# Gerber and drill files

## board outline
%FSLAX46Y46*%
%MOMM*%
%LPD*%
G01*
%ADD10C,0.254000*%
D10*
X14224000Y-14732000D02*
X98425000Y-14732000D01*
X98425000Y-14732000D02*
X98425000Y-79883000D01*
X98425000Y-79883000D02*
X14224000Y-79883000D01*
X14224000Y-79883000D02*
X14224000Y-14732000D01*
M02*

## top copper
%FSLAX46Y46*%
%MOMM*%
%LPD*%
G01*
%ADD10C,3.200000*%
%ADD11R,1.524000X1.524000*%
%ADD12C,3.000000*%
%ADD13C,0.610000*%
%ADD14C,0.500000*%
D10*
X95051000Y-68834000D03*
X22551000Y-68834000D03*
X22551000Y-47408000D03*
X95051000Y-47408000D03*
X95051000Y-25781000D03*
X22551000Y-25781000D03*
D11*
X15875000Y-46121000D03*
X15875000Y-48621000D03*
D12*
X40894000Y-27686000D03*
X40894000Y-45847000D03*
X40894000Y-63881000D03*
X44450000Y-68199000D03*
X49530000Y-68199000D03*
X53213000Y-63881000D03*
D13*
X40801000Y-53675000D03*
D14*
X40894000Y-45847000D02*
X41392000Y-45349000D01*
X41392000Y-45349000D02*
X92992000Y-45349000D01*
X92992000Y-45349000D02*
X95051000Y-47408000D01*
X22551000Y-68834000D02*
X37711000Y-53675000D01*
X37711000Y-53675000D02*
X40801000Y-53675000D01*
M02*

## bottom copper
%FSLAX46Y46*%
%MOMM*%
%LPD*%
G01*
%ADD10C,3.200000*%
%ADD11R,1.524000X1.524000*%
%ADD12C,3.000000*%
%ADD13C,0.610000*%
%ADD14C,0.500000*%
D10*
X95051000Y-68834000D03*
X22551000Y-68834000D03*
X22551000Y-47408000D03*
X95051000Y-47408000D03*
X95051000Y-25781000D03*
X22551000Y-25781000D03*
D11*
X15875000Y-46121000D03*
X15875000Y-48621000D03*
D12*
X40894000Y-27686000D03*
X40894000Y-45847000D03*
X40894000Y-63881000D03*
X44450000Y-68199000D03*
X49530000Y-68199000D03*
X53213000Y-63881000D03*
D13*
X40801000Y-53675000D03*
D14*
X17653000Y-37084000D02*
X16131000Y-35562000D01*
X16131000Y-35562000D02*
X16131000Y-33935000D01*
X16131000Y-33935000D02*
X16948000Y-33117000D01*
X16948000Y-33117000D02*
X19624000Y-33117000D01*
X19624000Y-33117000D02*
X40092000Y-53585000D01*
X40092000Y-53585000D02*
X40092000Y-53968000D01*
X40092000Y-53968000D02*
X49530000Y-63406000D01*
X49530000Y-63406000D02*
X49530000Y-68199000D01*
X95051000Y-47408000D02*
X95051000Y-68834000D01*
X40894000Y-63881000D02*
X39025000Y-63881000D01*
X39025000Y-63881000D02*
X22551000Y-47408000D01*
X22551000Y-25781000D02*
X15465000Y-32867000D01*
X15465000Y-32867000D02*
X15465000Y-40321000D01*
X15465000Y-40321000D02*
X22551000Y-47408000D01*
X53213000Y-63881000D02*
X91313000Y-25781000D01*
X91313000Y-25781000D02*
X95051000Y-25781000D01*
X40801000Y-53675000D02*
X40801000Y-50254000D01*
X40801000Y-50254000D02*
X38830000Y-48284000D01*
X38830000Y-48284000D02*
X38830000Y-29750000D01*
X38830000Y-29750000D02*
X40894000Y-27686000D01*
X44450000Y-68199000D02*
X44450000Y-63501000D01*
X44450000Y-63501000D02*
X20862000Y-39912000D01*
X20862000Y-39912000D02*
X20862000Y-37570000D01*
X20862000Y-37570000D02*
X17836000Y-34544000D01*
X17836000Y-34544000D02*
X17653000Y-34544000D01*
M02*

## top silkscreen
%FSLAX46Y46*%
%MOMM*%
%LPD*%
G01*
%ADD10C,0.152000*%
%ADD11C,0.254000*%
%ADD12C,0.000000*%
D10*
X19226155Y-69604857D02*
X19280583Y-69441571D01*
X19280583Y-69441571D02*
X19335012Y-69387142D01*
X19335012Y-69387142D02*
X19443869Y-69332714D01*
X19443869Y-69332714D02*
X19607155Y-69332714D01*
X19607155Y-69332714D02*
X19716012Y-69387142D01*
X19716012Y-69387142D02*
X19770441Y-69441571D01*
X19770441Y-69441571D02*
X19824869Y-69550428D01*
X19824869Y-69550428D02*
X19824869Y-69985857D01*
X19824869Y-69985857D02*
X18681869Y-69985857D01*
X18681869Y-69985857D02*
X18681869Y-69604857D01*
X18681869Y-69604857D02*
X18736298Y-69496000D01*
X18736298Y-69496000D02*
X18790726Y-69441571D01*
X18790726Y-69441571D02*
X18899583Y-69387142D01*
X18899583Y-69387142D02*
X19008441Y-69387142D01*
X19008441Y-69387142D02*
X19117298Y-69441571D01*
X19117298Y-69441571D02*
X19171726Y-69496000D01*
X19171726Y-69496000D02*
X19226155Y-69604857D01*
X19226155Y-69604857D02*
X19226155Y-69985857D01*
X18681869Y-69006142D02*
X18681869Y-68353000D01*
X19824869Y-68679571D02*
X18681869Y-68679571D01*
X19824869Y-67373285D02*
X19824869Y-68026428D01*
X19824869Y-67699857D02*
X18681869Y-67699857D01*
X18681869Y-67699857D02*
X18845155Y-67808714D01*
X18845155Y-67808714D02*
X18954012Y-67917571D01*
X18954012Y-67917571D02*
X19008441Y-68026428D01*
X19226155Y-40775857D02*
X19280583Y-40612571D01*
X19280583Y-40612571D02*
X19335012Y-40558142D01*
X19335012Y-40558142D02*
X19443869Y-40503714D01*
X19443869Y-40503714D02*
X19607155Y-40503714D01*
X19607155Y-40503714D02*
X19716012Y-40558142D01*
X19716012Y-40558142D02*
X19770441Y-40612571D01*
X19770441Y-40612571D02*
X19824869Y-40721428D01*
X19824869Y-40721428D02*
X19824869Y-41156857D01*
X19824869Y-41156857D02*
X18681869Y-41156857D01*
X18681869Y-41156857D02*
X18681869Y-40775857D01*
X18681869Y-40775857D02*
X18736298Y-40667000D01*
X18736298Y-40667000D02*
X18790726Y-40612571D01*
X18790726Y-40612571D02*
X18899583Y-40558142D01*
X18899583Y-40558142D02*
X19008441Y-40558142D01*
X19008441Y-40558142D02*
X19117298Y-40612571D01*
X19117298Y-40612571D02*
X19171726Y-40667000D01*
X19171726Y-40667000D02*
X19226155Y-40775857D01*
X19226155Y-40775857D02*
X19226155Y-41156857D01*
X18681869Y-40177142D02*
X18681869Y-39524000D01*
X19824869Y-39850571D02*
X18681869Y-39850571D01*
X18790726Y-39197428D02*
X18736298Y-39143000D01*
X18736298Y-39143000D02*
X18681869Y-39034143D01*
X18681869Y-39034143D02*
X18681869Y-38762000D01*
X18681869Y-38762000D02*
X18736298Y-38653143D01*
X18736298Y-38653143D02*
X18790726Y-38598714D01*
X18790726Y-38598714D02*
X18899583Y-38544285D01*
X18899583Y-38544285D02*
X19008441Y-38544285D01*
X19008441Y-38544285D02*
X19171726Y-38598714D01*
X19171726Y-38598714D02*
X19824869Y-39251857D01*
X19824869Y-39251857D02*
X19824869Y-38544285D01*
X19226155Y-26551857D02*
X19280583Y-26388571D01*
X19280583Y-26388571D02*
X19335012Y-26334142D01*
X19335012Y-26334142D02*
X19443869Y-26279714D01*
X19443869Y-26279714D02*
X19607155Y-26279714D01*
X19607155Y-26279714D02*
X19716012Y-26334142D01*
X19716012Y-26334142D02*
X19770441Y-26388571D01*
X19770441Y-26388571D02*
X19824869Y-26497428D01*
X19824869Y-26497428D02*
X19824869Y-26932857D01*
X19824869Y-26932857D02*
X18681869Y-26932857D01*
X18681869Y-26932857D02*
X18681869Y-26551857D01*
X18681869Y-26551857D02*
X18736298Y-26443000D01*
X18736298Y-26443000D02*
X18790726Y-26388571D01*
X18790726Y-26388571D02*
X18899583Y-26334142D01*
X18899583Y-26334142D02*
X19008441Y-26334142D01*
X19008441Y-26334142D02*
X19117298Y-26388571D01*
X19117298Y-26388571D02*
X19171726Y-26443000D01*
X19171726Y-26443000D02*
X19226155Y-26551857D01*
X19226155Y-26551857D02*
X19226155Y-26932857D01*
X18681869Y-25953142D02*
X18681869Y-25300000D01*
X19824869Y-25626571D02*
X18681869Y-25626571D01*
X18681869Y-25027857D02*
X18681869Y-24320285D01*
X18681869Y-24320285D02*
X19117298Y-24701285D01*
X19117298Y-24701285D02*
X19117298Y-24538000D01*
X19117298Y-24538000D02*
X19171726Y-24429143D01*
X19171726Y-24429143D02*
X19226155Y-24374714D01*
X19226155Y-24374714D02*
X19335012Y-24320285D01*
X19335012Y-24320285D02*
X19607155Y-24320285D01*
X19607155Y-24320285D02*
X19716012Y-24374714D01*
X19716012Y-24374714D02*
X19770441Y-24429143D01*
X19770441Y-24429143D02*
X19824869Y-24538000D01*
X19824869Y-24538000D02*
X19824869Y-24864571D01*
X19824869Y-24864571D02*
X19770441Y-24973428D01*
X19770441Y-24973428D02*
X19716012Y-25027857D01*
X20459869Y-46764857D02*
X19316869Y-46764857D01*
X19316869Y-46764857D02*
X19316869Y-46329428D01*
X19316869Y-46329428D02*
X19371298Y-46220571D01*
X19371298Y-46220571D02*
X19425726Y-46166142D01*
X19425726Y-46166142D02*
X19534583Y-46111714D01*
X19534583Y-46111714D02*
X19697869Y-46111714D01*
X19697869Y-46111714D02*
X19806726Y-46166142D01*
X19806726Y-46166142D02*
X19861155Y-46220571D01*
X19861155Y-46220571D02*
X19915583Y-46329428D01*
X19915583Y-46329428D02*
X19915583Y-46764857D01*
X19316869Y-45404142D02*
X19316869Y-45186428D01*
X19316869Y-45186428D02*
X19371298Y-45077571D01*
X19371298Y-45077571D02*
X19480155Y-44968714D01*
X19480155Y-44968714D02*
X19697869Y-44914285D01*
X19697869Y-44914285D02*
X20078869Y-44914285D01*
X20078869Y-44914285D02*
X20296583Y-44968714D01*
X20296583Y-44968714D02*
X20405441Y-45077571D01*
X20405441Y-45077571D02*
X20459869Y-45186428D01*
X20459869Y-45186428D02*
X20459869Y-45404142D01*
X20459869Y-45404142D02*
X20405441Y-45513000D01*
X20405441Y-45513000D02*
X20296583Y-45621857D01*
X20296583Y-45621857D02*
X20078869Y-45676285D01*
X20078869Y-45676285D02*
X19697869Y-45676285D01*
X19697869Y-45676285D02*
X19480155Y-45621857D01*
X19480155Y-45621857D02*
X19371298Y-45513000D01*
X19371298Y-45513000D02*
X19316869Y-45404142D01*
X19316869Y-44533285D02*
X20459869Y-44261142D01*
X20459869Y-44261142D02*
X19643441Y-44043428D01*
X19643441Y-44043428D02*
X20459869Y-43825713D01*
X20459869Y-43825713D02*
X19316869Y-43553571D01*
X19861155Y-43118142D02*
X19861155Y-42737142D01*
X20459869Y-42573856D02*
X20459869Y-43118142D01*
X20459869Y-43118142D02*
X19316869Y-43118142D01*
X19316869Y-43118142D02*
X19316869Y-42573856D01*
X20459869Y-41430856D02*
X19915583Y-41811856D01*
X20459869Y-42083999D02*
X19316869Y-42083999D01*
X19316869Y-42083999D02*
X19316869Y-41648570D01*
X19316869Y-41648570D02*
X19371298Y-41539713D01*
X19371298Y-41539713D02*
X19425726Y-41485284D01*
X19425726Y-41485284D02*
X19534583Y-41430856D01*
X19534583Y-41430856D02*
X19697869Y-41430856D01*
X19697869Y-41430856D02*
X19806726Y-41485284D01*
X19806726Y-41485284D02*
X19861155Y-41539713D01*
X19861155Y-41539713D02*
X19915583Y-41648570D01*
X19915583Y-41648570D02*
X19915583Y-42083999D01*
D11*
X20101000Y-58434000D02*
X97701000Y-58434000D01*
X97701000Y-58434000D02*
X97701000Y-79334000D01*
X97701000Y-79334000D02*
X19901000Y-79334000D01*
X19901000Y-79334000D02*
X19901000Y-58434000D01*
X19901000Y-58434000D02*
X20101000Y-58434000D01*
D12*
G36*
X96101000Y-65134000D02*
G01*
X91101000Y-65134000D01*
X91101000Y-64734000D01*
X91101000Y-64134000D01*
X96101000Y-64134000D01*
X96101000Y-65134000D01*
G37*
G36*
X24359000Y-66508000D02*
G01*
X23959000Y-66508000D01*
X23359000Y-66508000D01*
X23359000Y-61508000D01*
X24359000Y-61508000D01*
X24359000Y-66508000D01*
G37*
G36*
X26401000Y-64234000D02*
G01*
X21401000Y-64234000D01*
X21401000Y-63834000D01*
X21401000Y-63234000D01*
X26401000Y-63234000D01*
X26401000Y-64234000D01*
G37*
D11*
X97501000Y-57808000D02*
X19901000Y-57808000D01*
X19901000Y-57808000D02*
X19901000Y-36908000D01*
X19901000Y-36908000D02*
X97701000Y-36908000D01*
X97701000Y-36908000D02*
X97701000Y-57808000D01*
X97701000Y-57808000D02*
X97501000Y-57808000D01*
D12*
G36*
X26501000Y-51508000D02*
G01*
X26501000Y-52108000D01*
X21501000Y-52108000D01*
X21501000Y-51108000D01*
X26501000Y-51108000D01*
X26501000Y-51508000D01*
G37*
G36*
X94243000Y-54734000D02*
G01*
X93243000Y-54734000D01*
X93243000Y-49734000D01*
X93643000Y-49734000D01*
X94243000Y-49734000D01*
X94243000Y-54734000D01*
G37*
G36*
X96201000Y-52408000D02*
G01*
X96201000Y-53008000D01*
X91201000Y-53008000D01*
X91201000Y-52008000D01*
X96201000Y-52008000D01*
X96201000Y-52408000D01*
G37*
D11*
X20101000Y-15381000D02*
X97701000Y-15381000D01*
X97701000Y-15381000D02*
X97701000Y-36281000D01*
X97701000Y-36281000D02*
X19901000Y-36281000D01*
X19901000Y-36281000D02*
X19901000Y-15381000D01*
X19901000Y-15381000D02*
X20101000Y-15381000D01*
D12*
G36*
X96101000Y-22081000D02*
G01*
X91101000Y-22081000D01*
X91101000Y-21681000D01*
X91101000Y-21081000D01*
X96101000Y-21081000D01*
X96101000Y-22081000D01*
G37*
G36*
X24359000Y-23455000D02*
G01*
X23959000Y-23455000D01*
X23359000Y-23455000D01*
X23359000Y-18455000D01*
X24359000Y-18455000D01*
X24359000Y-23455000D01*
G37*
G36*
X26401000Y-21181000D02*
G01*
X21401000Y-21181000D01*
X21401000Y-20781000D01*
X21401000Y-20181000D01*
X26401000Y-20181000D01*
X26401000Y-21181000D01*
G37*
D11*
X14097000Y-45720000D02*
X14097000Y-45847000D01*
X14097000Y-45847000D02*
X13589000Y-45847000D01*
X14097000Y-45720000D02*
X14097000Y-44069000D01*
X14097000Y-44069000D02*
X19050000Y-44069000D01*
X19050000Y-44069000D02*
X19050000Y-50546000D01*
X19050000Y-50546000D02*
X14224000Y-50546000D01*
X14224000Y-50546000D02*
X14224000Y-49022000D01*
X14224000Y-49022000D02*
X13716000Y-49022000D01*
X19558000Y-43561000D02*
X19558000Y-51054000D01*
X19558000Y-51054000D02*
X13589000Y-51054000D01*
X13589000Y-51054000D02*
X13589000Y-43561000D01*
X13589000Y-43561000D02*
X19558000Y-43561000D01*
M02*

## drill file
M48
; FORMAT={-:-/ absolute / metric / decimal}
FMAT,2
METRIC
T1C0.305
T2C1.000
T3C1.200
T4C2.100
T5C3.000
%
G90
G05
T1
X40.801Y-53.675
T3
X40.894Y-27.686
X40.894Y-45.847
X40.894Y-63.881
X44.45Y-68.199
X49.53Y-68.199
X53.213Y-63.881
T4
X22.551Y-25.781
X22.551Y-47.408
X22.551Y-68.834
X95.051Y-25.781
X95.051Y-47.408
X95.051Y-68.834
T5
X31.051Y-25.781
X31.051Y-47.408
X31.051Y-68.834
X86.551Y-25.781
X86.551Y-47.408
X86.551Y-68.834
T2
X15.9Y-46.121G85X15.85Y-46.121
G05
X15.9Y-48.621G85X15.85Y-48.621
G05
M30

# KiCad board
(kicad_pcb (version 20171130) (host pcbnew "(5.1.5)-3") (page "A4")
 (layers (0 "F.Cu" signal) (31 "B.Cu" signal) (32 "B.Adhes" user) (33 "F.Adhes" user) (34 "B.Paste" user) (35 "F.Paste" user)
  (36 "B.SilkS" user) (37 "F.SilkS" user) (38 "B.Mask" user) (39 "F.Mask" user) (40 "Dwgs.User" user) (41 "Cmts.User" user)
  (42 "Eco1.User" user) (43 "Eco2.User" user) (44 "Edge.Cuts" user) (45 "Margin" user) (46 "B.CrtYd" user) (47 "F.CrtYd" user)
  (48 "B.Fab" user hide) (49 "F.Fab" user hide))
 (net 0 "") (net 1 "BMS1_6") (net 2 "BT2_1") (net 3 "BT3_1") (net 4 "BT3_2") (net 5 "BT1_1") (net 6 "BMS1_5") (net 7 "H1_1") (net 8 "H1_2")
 (segment (start 17.653 37.084) (end 16.131 35.562) (width 0.5) (layer "B.Cu") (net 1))
 (segment (start 16.131 35.562) (end 16.131 33.935) (width 0.5) (layer "B.Cu") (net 1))
 (segment (start 16.131 33.935) (end 16.948 33.117) (width 0.5) (layer "B.Cu") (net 1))
 (segment (start 16.948 33.117) (end 19.624 33.117) (width 0.5) (layer "B.Cu") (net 1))
 (segment (start 19.624 33.117) (end 40.092 53.585) (width 0.5) (layer "B.Cu") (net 1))
 (segment (start 40.092 53.585) (end 40.092 53.968) (width 0.5) (layer "B.Cu") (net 1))
 (segment (start 40.092 53.968) (end 49.53 63.406) (width 0.5) (layer "B.Cu") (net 1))
 (segment (start 49.53 63.406) (end 49.53 68.199) (width 0.5) (layer "B.Cu") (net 1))
 (segment (start 95.051 47.408) (end 95.051 68.834) (width 0.5) (layer "B.Cu") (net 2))
 (segment (start 40.894 63.881) (end 39.025 63.881) (width 0.5) (layer "B.Cu") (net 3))
 (segment (start 39.025 63.881) (end 22.551 47.408) (width 0.5) (layer "B.Cu") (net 3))
 (segment (start 22.551 25.781) (end 15.465 32.867) (width 0.5) (layer "B.Cu") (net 3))
 (segment (start 15.465 32.867) (end 15.465 40.321) (width 0.5) (layer "B.Cu") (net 3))
 (segment (start 15.465 40.321) (end 22.551 47.408) (width 0.5) (layer "B.Cu") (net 3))
 (segment (start 53.213 63.881) (end 91.313 25.781) (width 0.5) (layer "B.Cu") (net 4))
 (segment (start 91.313 25.781) (end 95.051 25.781) (width 0.5) (layer "B.Cu") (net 4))
 (segment (start 40.801 53.675) (end 40.801 50.254) (width 0.5) (layer "B.Cu") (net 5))
 (segment (start 40.801 50.254) (end 38.83 48.284) (width 0.5) (layer "B.Cu") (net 5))
 (segment (start 38.83 48.284) (end 38.83 29.75) (width 0.5) (layer "B.Cu") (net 5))
 (segment (start 38.83 29.75) (end 40.894 27.686) (width 0.5) (layer "B.Cu") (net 5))
 (segment (start 44.45 68.199) (end 44.45 63.501) (width 0.5) (layer "B.Cu") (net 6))
 (segment (start 44.45 63.501) (end 20.862 39.912) (width 0.5) (layer "B.Cu") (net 6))
 (segment (start 20.862 39.912) (end 20.862 37.57) (width 0.5) (layer "B.Cu") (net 6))
 (segment (start 20.862 37.57) (end 17.836 34.544) (width 0.5) (layer "B.Cu") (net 6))
 (segment (start 17.836 34.544) (end 17.653 34.544) (width 0.5) (layer "B.Cu") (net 6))
 (gr_line (start 14.224 14.732) (end 98.425 14.732) (width 0.254) (layer "Edge.Cuts"))
 (gr_line (start 98.425 14.732) (end 98.425 79.883) (width 0.254) (layer "Edge.Cuts"))
 (gr_line (start 98.425 79.883) (end 14.224 79.883) (width 0.254) (layer "Edge.Cuts"))
 (gr_line (start 14.224 79.883) (end 14.224 14.732) (width 0.254) (layer "Edge.Cuts"))
 (segment (start 40.894 45.847) (end 41.392 45.349) (width 0.5) (layer "F.Cu") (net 2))
 (segment (start 41.392 45.349) (end 92.992 45.349) (width 0.5) (layer "F.Cu") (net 2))
 (segment (start 92.992 45.349) (end 95.051 47.408) (width 0.5) (layer "F.Cu") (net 2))
 (segment (start 22.551 68.834) (end 37.711 53.675) (width 0.5) (layer "F.Cu") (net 5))
 (segment (start 37.711 53.675) (end 40.801 53.675) (width 0.5) (layer "F.Cu") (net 5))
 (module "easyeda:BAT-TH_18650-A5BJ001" (layer "F.Cu") (at 58.801 68.834)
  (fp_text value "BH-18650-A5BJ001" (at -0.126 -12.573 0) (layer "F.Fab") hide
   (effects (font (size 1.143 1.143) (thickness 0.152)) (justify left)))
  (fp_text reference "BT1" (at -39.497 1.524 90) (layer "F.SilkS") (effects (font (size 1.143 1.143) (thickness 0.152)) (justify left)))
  (fp_line (start -38.7 -10.4) (end 38.9 -10.4) (width 0.254) (layer "F.SilkS"))
  (fp_line (start 38.9 -10.4) (end 38.9 10.5) (width 0.254) (layer "F.SilkS"))
  (fp_line (start 38.9 10.5) (end -38.9 10.5) (width 0.254) (layer "F.SilkS"))
  (fp_line (start -38.9 10.5) (end -38.9 -10.4) (width 0.254) (layer "F.SilkS"))
  (fp_line (start -38.9 -10.4) (end -38.7 -10.4) (width 0.254) (layer "F.SilkS"))
  (fp_poly (pts (xy 32.3 -4.7) (xy 37.3 -4.7) (xy 37.3 -3.7) (xy 32.3 -3.7) (xy 32.3 -4.1)) (layer "F.SilkS") (width 0))
  (fp_poly
   (pts (xy -35.442 -2.326) (xy -35.442 -7.326) (xy -34.442 -7.326) (xy -34.442 -2.326) (xy -34.842 -2.326)) (layer "F.SilkS") (width 0))
  (fp_poly (pts (xy -37.4 -5.6) (xy -32.4 -5.6) (xy -32.4 -4.6) (xy -37.4 -4.6) (xy -37.4 -5)) (layer "F.SilkS") (width 0))
  (pad "" np_thru_hole circle (at 27.75 0) (size 3 3) (drill 3) (layers "*.Cu" "*.Mask"))
  (pad "" np_thru_hole circle (at -27.75 0) (size 3 3) (drill 3) (layers "*.Cu" "*.Mask"))
  (pad 2 thru_hole circle (at 36.25 0 0) (size 3.2 3.2) (layers "*.Cu" "*.Paste" "*.Mask") (drill 2.1) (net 2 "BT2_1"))
  (pad 1 thru_hole circle (at -36.25 0 0) (size 3.2 3.2) (layers "*.Cu" "*.Paste" "*.Mask") (drill 2.1) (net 5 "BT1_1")))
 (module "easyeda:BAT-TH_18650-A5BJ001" (layer "F.Cu") (at 58.801 47.408 180)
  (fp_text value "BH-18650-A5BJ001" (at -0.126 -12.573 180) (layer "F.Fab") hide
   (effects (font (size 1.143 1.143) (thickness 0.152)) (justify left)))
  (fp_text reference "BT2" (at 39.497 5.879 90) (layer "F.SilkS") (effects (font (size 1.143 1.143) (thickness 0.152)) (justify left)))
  (fp_line (start -38.7 -10.4) (end 38.9 -10.4) (width 0.254) (layer "F.SilkS"))
  (fp_line (start 38.9 -10.4) (end 38.9 10.5) (width 0.254) (layer "F.SilkS"))
  (fp_line (start 38.9 10.5) (end -38.9 10.5) (width 0.254) (layer "F.SilkS"))
  (fp_line (start -38.9 10.5) (end -38.9 -10.4) (width 0.254) (layer "F.SilkS"))
  (fp_line (start -38.9 -10.4) (end -38.7 -10.4) (width 0.254) (layer "F.SilkS"))
  (fp_poly (pts (xy 32.3 -4.7) (xy 37.3 -4.7) (xy 37.3 -3.7) (xy 32.3 -3.7) (xy 32.3 -4.1)) (layer "F.SilkS") (width 0))
  (fp_poly
   (pts (xy -35.442 -2.326) (xy -35.442 -7.326) (xy -34.442 -7.326) (xy -34.442 -2.326) (xy -34.842 -2.326)) (layer "F.SilkS") (width 0))
  (fp_poly (pts (xy -37.4 -5.6) (xy -32.4 -5.6) (xy -32.4 -4.6) (xy -37.4 -4.6) (xy -37.4 -5)) (layer "F.SilkS") (width 0))
  (pad "" np_thru_hole circle (at 27.75 0) (size 3 3) (drill 3) (layers "*.Cu" "*.Mask"))
  (pad "" np_thru_hole circle (at -27.75 0) (size 3 3) (drill 3) (layers "*.Cu" "*.Mask"))
  (pad 2 thru_hole circle (at 36.25 0 180) (size 3.2 3.2) (layers "*.Cu" "*.Paste" "*.Mask") (drill 2.1) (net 3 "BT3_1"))
  (pad 1 thru_hole circle (at -36.25 0 180) (size 3.2 3.2) (layers "*.Cu" "*.Paste" "*.Mask") (drill 2.1) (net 2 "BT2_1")))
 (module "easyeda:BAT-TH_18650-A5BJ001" (layer "F.Cu") (at 58.801 25.781)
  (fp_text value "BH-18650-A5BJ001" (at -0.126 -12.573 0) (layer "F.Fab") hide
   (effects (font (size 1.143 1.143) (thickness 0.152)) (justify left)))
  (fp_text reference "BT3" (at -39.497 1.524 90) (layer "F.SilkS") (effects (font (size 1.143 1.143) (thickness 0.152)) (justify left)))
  (fp_line (start -38.7 -10.4) (end 38.9 -10.4) (width 0.254) (layer "F.SilkS"))
  (fp_line (start 38.9 -10.4) (end 38.9 10.5) (width 0.254) (layer "F.SilkS"))
  (fp_line (start 38.9 10.5) (end -38.9 10.5) (width 0.254) (layer "F.SilkS"))
  (fp_line (start -38.9 10.5) (end -38.9 -10.4) (width 0.254) (layer "F.SilkS"))
  (fp_line (start -38.9 -10.4) (end -38.7 -10.4) (width 0.254) (layer "F.SilkS"))
  (fp_poly (pts (xy 32.3 -4.7) (xy 37.3 -4.7) (xy 37.3 -3.7) (xy 32.3 -3.7) (xy 32.3 -4.1)) (layer "F.SilkS") (width 0))
  (fp_poly
   (pts (xy -35.442 -2.326) (xy -35.442 -7.326) (xy -34.442 -7.326) (xy -34.442 -2.326) (xy -34.842 -2.326)) (layer "F.SilkS") (width 0))
  (fp_poly (pts (xy -37.4 -5.6) (xy -32.4 -5.6) (xy -32.4 -4.6) (xy -37.4 -4.6) (xy -37.4 -5)) (layer "F.SilkS") (width 0))
  (pad "" np_thru_hole circle (at 27.75 0) (size 3 3) (drill 3) (layers "*.Cu" "*.Mask"))
  (pad "" np_thru_hole circle (at -27.75 0) (size 3 3) (drill 3) (layers "*.Cu" "*.Mask"))
  (pad 2 thru_hole circle (at 36.25 0 0) (size 3.2 3.2) (layers "*.Cu" "*.Paste" "*.Mask") (drill 2.1) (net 4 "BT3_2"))
  (pad 1 thru_hole circle (at -36.25 0 0) (size 3.2 3.2) (layers "*.Cu" "*.Paste" "*.Mask") (drill 2.1) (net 3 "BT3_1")))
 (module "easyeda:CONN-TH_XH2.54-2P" (layer "F.Cu") (at 15.875 47.371 -90)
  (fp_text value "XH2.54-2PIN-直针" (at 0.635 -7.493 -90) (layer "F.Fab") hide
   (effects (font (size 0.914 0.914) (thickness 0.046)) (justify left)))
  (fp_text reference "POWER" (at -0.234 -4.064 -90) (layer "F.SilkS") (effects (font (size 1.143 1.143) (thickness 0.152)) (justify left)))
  (fp_line (start -1.651 1.778) (end -1.524 1.778) (width 0.254) (layer "F.SilkS"))
  (fp_line (start -1.524 1.778) (end -1.524 2.286) (width 0.254) (layer "F.SilkS"))
  (fp_line (start -1.651 1.778) (end -3.302 1.778) (width 0.254) (layer "F.SilkS"))
  (fp_line (start -3.302 1.778) (end -3.302 -3.175) (width 0.254) (layer "F.SilkS"))
  (fp_line (start -3.302 -3.175) (end 3.175 -3.175) (width 0.254) (layer "F.SilkS"))
  (fp_line (start 3.175 -3.175) (end 3.175 1.651) (width 0.254) (layer "F.SilkS"))
  (fp_line (start 3.175 1.651) (end 1.651 1.651) (width 0.254) (layer "F.SilkS"))
  (fp_line (start 1.651 1.651) (end 1.651 2.159) (width 0.254) (layer "F.SilkS"))
  (fp_line (start -3.81 -3.683) (end 3.683 -3.683) (width 0.254) (layer "F.SilkS"))
  (fp_line (start 3.683 -3.683) (end 3.683 2.286) (width 0.254) (layer "F.SilkS"))
  (fp_line (start 3.683 2.286) (end -3.81 2.286) (width 0.254) (layer "F.SilkS"))
  (fp_line (start -3.81 2.286) (end -3.81 -3.683) (width 0.254) (layer "F.SilkS"))
  (pad 1 thru_hole rect (at -1.25 0 -90) (size 1.524 1.524) (layers "*.Cu" "*.Paste" "*.Mask") (drill oval 1 1.05) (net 1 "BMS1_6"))
  (pad 2 thru_hole rect (at 1.25 0 -90) (size 1.524 1.524) (layers "*.Cu" "*.Paste" "*.Mask") (drill oval 1 1.05) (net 6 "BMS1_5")))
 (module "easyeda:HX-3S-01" (layer "F.Cu") (at 38.989 20.828 90)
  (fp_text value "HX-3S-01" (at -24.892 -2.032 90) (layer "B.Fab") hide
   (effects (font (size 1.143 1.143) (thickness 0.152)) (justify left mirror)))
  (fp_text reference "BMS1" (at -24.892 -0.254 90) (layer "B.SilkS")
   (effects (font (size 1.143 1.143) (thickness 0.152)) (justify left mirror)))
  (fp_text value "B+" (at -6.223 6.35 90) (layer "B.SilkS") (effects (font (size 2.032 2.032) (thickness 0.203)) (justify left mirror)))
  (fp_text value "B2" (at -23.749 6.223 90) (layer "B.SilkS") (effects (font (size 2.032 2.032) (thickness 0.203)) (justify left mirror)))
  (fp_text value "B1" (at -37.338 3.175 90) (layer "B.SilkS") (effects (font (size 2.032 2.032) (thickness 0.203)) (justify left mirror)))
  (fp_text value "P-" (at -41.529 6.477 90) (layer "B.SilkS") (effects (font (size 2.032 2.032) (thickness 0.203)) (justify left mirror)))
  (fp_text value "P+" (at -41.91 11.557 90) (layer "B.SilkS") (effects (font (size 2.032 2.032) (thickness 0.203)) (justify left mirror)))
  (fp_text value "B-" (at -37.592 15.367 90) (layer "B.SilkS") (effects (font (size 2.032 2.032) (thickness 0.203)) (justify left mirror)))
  (pad 1 thru_hole circle (at -6.858 1.905 90) (size 3 3) (layers "*.Cu" "*.Paste" "*.Mask") (drill 1.2) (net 5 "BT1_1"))
  (pad 2 thru_hole circle (at -25.019 1.905 90) (size 3 3) (layers "*.Cu" "*.Paste" "*.Mask") (drill 1.2) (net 2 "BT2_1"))
  (pad 3 thru_hole circle (at -43.053 1.905 90) (size 3 3) (layers "*.Cu" "*.Paste" "*.Mask") (drill 1.2) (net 3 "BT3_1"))
  (pad 5 thru_hole circle (at -47.371 5.461 90) (size 3 3) (layers "*.Cu" "*.Paste" "*.Mask") (drill 1.2) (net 6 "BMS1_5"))
  (pad 6 thru_hole circle (at -47.371 10.541 90) (size 3 3) (layers "*.Cu" "*.Paste" "*.Mask") (drill 1.2) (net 1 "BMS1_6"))
  (pad 4 thru_hole circle (at -43.053 14.224 90) (size 3 3) (layers "*.Cu" "*.Paste" "*.Mask") (drill 1.2) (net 4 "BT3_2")))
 (via (at 40.801 53.675) (size 0.61) (drill 0.305) (layers "F.Cu" "B.Cu") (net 5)))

